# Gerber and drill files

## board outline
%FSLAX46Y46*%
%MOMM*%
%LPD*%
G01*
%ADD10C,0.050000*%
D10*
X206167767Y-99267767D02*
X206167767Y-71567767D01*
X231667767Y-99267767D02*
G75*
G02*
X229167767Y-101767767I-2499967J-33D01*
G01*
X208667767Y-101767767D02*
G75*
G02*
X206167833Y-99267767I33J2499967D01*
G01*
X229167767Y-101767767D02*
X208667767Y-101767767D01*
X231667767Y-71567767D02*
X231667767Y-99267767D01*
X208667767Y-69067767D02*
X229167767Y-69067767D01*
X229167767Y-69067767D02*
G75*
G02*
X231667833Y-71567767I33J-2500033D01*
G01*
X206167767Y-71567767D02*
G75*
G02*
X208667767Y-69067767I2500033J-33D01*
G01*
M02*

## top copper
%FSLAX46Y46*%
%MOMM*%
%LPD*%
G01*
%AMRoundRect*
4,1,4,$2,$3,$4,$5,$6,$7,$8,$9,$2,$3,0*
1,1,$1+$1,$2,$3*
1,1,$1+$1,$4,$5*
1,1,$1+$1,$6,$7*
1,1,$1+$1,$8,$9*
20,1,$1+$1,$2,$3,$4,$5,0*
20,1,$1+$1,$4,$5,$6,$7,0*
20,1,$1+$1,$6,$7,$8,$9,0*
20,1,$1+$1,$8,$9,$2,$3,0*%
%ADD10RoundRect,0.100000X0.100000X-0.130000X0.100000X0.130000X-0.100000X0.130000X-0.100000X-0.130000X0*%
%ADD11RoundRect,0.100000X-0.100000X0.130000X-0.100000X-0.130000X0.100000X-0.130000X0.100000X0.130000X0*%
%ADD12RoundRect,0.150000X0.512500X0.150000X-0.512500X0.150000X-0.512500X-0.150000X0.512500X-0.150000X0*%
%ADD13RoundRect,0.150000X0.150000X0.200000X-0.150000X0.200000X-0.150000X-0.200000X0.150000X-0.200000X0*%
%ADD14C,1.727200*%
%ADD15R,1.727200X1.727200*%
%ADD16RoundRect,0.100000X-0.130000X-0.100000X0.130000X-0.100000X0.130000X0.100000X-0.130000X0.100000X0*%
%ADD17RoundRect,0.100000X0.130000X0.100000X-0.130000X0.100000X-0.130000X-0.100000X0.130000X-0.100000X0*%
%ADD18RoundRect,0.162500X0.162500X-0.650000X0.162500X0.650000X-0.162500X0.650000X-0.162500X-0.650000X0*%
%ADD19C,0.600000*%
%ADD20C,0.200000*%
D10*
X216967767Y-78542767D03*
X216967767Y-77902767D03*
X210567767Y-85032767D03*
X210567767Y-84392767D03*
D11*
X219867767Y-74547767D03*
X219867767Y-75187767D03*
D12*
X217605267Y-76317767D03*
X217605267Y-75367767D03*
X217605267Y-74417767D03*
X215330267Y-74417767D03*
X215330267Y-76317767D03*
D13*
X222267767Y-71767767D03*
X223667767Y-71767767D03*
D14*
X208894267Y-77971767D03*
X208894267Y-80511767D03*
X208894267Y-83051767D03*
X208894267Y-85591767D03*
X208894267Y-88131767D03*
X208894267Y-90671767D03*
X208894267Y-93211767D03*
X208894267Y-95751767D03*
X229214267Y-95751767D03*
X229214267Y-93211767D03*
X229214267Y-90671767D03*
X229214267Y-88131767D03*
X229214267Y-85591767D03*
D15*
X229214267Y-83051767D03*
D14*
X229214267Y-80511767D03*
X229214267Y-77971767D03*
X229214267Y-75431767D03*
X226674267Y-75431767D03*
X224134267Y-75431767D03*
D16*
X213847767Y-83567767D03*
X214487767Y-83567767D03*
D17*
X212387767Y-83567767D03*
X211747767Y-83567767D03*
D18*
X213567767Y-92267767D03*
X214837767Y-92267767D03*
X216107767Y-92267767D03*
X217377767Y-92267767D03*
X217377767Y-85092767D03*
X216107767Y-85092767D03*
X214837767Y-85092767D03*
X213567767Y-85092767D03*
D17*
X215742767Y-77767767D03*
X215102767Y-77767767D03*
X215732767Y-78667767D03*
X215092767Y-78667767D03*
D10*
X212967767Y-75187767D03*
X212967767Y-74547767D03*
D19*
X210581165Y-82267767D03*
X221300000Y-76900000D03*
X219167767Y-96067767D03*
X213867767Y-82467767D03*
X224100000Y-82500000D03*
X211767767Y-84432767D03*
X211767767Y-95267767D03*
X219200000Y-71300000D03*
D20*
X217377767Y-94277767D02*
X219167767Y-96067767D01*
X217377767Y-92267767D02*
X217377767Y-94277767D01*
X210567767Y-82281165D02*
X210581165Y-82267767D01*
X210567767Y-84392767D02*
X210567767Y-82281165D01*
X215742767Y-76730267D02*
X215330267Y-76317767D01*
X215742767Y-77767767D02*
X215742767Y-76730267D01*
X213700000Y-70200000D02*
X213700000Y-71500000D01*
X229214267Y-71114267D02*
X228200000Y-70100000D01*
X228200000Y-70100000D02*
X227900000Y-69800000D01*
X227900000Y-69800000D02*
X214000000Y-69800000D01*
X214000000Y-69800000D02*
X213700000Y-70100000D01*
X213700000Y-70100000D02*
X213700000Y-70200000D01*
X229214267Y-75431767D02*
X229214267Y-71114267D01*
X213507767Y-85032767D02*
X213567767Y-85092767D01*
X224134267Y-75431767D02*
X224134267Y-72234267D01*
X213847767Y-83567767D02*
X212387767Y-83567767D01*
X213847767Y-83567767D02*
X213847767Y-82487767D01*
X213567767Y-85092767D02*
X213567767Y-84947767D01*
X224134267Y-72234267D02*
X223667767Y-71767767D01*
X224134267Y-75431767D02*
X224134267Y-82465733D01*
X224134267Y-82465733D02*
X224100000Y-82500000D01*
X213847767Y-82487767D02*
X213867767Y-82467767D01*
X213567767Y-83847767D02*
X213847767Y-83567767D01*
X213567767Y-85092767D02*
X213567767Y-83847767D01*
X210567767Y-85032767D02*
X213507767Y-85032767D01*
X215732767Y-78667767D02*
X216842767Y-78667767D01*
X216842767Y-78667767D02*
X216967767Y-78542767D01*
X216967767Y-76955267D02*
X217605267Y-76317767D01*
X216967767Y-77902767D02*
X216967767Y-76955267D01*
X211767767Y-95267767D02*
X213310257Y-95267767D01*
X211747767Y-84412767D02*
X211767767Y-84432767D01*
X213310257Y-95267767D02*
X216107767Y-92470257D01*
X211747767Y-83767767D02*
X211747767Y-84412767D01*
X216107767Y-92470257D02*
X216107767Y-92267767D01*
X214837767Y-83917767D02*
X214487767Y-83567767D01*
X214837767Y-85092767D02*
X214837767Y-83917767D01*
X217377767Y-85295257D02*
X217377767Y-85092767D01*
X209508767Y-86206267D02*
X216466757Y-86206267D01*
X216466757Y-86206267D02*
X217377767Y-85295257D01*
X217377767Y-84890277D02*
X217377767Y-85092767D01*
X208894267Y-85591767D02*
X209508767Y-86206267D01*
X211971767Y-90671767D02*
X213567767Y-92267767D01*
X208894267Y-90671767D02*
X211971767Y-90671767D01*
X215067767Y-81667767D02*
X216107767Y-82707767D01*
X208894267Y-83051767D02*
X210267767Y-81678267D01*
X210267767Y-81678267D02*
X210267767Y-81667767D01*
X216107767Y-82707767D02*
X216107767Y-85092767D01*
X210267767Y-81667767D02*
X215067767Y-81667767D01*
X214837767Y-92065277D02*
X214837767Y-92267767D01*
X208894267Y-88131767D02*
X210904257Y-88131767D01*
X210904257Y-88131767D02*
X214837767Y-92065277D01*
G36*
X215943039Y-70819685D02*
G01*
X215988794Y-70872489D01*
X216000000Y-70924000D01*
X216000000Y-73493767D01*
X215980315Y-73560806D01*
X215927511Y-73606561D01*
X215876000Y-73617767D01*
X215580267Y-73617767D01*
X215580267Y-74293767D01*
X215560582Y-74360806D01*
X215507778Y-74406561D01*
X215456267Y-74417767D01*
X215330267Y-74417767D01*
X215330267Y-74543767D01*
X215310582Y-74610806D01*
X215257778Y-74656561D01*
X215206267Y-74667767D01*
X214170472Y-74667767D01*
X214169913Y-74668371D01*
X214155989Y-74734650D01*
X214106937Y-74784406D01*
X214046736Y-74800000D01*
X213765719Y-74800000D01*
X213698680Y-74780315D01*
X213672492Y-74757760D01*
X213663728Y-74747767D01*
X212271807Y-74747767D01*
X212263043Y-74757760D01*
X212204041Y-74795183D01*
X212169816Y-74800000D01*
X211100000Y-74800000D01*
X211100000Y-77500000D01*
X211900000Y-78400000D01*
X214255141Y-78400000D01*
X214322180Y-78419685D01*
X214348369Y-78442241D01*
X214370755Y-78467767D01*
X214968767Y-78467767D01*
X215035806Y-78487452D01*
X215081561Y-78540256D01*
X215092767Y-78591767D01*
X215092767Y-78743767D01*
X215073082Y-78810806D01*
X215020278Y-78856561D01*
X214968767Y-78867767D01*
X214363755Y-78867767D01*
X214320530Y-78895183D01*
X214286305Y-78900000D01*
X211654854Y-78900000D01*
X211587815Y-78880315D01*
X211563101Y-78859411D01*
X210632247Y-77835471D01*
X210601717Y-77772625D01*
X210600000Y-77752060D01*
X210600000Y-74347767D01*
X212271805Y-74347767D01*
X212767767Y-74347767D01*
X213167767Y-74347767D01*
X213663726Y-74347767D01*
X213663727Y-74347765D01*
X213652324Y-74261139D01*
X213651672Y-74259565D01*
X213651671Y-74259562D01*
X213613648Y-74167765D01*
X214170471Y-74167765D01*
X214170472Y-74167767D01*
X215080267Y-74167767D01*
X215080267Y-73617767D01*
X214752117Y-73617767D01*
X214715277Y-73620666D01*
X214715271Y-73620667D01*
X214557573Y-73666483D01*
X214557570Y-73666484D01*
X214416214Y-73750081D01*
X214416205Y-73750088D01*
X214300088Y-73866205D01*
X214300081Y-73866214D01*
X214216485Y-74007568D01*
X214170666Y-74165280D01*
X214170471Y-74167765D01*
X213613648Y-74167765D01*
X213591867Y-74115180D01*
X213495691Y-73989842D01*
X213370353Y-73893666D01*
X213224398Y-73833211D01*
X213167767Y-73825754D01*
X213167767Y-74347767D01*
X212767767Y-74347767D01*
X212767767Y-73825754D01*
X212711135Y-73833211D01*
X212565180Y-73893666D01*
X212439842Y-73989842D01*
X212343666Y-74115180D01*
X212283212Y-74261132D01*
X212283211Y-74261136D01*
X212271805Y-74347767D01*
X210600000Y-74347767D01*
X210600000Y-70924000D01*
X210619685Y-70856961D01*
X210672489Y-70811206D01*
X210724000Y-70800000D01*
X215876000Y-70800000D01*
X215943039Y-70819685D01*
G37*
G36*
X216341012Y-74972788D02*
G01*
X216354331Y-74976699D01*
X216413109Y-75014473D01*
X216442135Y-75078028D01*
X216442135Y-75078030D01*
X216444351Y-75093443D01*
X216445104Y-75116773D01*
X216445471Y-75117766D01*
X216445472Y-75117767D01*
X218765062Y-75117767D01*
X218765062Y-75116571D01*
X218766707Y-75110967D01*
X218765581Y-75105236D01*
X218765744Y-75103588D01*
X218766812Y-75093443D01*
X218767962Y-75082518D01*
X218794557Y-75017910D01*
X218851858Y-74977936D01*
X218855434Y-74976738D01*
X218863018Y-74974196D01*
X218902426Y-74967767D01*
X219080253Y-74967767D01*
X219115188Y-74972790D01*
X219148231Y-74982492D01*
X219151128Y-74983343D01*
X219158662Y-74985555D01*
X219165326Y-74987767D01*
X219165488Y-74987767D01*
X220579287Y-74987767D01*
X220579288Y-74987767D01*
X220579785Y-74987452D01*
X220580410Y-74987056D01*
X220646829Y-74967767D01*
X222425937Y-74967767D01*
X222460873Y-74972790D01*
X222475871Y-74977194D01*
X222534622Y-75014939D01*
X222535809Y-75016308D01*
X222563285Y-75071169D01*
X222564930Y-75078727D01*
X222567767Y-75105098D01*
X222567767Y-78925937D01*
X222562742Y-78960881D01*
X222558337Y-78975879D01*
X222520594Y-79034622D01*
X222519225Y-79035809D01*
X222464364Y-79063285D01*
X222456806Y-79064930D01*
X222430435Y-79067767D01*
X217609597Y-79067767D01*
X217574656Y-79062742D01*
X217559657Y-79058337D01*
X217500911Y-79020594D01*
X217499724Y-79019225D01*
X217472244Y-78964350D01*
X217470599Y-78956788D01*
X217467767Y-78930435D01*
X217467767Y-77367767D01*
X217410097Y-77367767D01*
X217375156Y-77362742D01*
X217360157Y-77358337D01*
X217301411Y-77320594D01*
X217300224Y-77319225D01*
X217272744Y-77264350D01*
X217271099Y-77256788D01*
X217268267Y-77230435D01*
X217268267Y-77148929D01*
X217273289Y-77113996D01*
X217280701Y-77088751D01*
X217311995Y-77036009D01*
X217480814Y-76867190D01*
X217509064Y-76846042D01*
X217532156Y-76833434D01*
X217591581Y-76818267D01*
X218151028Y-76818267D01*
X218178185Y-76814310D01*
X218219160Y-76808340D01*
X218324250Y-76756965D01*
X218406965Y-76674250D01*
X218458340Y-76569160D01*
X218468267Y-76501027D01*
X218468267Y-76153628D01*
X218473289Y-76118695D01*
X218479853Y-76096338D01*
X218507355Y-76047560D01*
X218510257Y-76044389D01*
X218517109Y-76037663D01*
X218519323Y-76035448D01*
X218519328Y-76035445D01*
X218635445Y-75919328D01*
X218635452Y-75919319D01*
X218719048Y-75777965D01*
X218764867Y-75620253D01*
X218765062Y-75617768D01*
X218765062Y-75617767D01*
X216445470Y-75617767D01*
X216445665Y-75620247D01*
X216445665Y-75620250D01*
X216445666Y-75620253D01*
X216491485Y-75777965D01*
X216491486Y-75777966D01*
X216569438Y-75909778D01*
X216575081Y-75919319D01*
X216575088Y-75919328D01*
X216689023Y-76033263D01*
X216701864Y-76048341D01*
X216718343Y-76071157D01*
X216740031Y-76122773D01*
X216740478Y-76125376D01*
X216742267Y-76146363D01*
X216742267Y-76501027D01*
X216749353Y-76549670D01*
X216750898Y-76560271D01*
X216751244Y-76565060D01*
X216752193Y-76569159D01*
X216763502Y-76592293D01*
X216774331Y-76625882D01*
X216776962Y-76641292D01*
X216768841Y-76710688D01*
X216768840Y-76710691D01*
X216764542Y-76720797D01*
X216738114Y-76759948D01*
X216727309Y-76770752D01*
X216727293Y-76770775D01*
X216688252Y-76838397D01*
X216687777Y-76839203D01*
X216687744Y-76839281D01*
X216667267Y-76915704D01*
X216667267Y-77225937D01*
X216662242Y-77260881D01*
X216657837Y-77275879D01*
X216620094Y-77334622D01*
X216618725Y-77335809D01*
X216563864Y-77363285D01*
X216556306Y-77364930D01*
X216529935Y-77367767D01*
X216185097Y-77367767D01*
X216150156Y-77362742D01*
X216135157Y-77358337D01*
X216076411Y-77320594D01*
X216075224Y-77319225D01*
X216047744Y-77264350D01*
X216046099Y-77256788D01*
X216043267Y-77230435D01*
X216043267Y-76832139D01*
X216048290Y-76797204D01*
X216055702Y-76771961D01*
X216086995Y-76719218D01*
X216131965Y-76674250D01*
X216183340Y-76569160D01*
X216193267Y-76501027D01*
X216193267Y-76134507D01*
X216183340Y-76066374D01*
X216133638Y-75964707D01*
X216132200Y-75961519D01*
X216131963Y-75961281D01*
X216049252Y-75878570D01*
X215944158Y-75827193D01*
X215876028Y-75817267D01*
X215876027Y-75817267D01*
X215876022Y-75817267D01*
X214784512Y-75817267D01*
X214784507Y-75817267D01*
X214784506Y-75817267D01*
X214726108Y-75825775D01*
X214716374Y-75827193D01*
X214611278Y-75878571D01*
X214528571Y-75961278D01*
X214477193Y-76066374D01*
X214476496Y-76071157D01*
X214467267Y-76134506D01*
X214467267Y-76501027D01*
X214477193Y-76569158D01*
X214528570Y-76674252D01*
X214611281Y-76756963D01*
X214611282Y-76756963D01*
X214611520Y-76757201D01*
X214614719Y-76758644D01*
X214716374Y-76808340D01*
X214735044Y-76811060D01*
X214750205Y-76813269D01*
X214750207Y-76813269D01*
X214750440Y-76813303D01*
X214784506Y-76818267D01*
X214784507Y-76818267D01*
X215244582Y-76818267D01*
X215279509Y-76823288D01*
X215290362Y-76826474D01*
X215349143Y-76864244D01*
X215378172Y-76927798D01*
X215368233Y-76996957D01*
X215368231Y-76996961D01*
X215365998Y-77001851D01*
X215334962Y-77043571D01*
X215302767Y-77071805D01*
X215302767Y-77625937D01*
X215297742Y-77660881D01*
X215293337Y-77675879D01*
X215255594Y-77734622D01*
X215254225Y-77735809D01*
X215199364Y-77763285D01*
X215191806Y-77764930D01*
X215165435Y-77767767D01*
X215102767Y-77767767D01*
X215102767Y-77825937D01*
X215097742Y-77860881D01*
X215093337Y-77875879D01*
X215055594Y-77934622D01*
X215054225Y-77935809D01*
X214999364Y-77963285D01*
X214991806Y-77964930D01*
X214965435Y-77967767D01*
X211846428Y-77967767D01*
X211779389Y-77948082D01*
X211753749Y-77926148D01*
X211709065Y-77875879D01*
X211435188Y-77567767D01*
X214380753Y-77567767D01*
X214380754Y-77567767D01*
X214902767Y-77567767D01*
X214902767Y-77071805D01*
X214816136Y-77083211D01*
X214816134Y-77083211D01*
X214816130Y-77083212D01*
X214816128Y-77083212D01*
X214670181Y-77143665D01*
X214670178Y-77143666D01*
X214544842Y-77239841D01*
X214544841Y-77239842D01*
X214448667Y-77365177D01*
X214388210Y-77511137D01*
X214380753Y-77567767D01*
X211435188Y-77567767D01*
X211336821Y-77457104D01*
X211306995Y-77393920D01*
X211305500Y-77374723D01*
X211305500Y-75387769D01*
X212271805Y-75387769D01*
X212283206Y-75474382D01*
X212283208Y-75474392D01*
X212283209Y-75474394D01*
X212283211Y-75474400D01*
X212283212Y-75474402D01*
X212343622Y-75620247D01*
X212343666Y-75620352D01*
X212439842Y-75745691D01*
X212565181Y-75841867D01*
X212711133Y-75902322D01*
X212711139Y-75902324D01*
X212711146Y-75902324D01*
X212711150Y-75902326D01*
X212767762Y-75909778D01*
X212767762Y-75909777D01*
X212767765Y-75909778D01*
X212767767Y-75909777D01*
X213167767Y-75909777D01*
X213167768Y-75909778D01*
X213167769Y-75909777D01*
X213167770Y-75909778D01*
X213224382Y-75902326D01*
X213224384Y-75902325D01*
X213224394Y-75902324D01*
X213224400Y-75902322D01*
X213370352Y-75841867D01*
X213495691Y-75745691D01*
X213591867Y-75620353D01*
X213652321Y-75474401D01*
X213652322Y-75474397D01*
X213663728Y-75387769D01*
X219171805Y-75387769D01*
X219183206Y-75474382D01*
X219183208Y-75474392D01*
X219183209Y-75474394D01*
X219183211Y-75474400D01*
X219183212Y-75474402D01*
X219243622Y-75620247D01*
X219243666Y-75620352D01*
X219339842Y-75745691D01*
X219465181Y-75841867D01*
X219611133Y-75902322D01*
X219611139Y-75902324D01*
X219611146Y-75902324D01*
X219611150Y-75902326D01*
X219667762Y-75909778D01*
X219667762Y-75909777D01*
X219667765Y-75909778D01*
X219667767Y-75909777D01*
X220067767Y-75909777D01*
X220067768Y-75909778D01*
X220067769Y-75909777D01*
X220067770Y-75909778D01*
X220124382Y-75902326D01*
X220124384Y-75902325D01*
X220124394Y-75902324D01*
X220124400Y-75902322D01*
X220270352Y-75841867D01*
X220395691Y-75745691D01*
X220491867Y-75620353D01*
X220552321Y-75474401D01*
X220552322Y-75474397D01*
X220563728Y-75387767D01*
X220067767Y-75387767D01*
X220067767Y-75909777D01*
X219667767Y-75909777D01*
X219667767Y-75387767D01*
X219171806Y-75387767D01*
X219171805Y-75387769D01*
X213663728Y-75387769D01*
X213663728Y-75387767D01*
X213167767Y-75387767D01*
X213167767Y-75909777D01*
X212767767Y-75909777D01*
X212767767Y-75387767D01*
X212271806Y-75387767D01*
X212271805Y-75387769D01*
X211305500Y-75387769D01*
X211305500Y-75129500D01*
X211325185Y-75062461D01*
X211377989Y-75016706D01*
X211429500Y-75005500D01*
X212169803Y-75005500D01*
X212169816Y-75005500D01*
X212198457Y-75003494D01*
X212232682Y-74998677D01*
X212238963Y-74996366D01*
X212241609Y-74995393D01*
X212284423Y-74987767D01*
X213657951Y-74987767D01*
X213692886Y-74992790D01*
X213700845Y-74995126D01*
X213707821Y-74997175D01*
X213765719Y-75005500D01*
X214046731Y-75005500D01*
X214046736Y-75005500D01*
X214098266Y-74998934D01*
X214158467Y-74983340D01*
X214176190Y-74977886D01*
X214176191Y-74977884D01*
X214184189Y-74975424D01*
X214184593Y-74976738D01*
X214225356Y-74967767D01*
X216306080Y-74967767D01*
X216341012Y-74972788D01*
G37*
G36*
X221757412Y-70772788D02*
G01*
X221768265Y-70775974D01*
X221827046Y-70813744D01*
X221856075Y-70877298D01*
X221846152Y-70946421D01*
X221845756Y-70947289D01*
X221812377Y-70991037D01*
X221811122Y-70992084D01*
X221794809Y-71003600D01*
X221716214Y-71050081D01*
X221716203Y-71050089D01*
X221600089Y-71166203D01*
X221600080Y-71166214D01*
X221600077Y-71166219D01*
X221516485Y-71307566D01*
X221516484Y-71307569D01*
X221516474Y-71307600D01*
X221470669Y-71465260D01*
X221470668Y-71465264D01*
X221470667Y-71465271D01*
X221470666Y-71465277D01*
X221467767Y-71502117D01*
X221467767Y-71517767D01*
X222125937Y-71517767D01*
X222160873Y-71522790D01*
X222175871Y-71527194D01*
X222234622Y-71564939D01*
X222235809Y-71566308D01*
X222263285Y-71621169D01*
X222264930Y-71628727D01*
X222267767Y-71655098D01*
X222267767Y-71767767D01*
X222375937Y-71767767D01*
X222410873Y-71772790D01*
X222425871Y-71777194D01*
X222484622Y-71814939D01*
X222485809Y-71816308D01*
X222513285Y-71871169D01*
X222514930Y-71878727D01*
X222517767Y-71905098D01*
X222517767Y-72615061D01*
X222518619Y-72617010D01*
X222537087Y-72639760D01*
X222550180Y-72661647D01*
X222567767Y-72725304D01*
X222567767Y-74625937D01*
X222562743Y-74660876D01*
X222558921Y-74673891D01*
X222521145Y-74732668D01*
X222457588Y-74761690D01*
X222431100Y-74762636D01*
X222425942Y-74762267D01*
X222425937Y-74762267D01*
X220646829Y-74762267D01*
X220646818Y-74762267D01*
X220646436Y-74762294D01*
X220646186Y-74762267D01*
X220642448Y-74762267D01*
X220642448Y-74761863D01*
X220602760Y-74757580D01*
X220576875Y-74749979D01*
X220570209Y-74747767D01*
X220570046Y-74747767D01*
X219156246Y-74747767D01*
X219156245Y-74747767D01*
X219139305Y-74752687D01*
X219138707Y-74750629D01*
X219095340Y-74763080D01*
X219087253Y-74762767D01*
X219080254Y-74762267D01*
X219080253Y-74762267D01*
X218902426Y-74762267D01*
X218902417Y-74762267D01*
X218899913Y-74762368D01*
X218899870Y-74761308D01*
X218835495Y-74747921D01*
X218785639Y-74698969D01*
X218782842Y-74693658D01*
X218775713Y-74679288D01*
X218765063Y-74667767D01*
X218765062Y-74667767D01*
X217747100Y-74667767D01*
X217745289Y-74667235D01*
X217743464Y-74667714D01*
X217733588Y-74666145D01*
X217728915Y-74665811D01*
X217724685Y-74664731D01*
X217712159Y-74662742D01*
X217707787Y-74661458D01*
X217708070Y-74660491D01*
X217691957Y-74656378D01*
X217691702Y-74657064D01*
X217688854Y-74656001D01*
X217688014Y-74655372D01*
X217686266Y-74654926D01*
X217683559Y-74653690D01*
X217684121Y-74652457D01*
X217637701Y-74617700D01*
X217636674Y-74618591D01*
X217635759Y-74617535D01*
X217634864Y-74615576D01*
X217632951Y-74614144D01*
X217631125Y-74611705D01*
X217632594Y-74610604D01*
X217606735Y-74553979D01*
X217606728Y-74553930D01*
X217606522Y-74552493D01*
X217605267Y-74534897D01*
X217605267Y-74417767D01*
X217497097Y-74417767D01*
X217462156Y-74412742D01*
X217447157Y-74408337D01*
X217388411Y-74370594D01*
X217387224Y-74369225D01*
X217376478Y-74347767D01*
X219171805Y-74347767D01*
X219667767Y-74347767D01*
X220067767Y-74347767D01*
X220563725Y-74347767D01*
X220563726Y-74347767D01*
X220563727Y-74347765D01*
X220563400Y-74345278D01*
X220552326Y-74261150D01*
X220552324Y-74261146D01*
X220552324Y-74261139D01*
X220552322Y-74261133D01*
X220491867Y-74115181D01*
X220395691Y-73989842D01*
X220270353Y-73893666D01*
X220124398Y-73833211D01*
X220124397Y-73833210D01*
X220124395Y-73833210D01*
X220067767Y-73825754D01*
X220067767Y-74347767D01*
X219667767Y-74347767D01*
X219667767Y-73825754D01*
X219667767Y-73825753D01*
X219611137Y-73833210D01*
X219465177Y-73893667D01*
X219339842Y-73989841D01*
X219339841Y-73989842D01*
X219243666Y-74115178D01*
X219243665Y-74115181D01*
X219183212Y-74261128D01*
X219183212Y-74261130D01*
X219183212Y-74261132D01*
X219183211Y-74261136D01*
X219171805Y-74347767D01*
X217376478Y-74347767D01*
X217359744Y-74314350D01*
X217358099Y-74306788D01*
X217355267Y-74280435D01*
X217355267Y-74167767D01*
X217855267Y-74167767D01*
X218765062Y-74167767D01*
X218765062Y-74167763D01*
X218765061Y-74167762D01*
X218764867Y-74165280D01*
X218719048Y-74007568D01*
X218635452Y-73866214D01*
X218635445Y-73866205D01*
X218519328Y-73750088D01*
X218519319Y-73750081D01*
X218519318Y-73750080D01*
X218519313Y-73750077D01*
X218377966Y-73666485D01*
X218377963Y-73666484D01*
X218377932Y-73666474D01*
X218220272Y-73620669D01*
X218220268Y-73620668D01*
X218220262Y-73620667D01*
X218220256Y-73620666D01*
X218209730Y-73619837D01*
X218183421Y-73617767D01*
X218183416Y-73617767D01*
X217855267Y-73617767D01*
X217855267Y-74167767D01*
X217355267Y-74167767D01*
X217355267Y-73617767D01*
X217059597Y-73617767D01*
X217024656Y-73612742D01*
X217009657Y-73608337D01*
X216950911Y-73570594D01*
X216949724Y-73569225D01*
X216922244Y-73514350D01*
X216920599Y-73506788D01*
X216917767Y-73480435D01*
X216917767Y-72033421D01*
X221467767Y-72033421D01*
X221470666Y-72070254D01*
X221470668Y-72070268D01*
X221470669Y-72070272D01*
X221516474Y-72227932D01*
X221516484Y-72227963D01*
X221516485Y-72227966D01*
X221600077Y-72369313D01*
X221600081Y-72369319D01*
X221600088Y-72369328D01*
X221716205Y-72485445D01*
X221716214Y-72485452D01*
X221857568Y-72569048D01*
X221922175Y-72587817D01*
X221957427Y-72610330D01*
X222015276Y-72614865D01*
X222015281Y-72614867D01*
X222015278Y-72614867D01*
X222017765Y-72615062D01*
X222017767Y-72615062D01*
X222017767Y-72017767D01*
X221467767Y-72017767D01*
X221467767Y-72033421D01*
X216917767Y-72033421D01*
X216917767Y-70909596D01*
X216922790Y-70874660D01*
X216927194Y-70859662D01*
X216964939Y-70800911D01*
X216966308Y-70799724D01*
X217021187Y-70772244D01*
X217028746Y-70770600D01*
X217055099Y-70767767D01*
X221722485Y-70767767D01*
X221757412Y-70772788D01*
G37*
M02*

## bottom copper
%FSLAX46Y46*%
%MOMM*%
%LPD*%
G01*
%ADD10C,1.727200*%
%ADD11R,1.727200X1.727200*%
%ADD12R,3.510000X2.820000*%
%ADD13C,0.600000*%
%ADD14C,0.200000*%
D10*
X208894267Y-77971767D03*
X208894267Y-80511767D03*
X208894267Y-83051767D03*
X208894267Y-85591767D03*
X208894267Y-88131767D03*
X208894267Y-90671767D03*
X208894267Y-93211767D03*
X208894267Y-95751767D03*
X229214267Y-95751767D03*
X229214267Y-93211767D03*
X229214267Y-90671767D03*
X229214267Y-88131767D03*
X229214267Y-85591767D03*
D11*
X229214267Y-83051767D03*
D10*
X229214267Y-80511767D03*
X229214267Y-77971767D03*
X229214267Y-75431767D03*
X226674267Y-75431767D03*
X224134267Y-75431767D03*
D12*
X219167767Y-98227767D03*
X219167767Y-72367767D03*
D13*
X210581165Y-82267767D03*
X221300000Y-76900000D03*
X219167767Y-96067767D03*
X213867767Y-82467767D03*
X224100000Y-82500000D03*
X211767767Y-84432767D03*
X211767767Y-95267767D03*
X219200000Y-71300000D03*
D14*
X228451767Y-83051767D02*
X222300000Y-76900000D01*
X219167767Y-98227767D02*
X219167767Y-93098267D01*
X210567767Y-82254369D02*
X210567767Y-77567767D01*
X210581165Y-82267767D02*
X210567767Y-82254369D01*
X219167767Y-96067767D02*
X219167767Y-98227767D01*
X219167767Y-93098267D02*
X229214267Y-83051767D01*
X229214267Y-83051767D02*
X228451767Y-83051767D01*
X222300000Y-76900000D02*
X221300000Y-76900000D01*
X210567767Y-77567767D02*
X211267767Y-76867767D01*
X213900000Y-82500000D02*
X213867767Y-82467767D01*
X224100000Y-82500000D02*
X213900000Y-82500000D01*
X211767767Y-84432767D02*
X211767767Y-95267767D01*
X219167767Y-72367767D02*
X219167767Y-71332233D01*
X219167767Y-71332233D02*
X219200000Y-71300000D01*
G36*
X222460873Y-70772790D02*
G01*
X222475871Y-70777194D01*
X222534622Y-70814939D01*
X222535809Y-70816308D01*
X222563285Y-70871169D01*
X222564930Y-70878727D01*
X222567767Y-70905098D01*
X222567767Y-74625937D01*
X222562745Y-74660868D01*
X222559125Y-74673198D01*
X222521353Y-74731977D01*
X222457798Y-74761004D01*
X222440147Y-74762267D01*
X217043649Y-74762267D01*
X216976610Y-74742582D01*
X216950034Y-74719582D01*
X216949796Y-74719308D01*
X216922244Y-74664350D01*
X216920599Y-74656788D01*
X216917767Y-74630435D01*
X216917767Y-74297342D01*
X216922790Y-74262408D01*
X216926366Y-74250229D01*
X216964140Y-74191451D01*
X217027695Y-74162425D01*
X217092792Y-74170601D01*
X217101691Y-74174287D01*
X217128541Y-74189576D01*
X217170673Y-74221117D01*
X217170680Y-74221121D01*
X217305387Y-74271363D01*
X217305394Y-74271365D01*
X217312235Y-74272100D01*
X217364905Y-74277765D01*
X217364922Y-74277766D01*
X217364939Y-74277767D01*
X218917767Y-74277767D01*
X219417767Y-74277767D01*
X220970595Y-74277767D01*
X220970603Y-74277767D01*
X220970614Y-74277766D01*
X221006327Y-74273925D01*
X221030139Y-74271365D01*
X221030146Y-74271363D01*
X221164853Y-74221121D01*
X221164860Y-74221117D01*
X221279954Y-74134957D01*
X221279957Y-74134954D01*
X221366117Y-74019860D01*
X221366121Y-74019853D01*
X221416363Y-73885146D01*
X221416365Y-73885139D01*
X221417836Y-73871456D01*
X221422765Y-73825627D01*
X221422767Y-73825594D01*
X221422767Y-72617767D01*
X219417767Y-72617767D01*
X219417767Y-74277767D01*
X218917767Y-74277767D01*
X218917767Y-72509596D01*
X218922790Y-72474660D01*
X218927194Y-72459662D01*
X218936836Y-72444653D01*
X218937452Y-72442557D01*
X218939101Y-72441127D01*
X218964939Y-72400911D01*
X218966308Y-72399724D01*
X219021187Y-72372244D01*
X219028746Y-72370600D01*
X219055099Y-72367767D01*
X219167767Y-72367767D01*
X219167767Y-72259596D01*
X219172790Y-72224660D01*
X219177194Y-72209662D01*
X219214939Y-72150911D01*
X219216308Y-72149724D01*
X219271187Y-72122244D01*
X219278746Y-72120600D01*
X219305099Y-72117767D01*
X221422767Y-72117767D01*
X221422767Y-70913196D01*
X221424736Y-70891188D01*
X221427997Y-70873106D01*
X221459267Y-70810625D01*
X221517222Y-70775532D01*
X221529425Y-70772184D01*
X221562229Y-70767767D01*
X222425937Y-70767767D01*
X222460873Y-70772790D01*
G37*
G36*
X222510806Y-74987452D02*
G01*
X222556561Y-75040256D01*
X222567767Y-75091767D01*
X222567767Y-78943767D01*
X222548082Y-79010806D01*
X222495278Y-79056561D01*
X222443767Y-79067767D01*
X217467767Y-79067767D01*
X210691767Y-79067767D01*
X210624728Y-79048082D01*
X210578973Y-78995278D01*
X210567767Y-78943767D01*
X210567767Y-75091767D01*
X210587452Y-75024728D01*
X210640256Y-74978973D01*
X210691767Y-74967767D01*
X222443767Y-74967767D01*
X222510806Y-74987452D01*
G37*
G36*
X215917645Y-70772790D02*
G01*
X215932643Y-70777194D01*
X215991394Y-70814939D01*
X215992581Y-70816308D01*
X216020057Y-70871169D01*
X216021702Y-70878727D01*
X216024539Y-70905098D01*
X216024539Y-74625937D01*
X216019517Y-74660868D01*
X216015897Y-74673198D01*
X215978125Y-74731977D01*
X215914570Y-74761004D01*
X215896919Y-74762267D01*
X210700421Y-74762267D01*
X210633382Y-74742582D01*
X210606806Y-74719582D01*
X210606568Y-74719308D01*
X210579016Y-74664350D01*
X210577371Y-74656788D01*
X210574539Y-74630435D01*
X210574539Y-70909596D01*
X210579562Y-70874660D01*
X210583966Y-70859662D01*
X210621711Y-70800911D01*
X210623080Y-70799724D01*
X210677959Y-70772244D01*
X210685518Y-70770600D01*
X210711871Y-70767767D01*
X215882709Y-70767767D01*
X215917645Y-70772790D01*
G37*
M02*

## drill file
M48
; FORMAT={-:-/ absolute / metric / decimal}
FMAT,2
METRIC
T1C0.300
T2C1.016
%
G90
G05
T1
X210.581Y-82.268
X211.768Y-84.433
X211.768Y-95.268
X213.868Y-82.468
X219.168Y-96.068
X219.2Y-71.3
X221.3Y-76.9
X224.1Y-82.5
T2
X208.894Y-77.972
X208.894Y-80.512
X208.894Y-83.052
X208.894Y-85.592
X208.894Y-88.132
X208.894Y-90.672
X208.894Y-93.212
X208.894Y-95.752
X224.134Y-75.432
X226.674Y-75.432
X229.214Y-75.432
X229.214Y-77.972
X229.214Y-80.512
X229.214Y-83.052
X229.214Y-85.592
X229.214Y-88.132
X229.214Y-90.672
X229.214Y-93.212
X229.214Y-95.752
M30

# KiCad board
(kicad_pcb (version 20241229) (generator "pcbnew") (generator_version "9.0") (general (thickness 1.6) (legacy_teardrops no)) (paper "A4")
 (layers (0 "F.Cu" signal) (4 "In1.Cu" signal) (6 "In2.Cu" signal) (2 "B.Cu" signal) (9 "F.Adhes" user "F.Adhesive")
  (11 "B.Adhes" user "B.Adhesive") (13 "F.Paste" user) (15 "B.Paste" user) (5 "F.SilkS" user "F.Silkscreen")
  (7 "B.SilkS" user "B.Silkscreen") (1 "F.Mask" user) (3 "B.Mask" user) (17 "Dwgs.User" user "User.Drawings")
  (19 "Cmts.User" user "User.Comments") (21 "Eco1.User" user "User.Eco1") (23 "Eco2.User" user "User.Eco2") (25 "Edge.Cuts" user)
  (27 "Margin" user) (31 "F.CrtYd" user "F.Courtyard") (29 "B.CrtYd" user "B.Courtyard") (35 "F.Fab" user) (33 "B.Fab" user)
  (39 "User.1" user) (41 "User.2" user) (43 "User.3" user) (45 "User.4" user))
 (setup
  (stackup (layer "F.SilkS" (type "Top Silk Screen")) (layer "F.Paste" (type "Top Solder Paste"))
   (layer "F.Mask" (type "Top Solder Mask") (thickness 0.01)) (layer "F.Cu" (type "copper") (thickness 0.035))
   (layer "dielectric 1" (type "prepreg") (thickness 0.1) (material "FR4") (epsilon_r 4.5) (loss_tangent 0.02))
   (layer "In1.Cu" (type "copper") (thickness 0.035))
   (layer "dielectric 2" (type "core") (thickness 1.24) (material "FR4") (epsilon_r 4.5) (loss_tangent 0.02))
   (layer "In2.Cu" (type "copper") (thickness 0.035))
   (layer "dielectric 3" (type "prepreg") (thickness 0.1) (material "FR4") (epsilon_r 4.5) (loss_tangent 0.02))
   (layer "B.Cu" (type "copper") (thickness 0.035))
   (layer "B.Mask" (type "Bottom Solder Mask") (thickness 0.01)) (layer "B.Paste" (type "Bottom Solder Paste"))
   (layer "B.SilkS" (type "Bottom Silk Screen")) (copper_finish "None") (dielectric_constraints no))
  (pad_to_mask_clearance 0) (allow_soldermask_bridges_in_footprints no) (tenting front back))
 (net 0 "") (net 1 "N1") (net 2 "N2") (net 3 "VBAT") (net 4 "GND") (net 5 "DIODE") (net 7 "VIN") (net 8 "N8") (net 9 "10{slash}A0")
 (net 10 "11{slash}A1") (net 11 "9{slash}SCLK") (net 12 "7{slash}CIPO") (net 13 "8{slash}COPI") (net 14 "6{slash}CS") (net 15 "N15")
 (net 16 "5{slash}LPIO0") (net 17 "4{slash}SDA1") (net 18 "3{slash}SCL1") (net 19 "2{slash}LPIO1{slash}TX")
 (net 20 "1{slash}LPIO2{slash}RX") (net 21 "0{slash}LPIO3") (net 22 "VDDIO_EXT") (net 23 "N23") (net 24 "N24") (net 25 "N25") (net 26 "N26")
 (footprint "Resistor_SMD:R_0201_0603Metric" (layer "F.Cu") (at 216.967767 78.222767 90)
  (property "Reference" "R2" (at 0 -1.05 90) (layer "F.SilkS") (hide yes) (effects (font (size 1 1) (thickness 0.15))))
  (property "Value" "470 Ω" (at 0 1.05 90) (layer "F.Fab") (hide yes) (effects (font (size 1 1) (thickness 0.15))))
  (pad "" smd roundrect (at -0.345 0 90) (size 0.318 0.36) (layers "F.Paste") (roundrect_rratio 0.25))
  (pad "" smd roundrect (at 0.345 0 90) (size 0.318 0.36) (layers "F.Paste") (roundrect_rratio 0.25))
  (pad "1" smd roundrect (at -0.32 0 90) (size 0.46 0.4) (layers "F.Cu" "F.Mask") (roundrect_rratio 0.25) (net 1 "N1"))
  (pad "2" smd roundrect (at 0.32 0 90) (size 0.46 0.4) (layers "F.Cu" "F.Mask") (roundrect_rratio 0.25) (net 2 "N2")))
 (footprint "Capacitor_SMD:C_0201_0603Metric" (layer "F.Cu") (at 210.567767 84.712767 90)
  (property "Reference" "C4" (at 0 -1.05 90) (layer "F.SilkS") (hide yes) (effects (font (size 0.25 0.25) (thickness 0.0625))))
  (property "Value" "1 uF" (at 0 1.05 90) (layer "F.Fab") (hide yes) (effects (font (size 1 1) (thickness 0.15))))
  (pad "" smd roundrect (at -0.345 0 90) (size 0.318 0.36) (layers "F.Paste") (roundrect_rratio 0.25))
  (pad "" smd roundrect (at 0.345 0 90) (size 0.318 0.36) (layers "F.Paste") (roundrect_rratio 0.25))
  (pad "1" smd roundrect (at -0.32 0 90) (size 0.46 0.4) (layers "F.Cu" "F.Mask") (roundrect_rratio 0.25) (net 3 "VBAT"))
  (pad "2" smd roundrect (at 0.32 0 90) (size 0.46 0.4) (layers "F.Cu" "F.Mask") (roundrect_rratio 0.25) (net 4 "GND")))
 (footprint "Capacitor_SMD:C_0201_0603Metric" (layer "F.Cu") (at 219.867767 74.867767 -90)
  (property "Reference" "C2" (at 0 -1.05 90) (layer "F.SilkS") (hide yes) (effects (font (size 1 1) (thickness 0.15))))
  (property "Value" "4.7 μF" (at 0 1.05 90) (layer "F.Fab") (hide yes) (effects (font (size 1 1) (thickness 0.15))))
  (pad "" smd roundrect (at -0.345 0 270) (size 0.318 0.36) (layers "F.Paste") (roundrect_rratio 0.25))
  (pad "" smd roundrect (at 0.345 0 270) (size 0.318 0.36) (layers "F.Paste") (roundrect_rratio 0.25))
  (pad "1" smd roundrect (at -0.32 0 270) (size 0.46 0.4) (layers "F.Cu" "F.Mask") (roundrect_rratio 0.25) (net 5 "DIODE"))
  (pad "2" smd roundrect (at 0.32 0 270) (size 0.46 0.4) (layers "F.Cu" "F.Mask") (roundrect_rratio 0.25) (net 4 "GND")))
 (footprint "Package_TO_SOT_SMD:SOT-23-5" (layer "F.Cu") (at 216.467767 75.367767 180)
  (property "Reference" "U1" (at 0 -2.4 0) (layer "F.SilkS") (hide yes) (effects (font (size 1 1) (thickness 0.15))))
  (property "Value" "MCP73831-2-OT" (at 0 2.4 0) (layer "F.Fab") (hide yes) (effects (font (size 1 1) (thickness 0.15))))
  (pad "1" smd roundrect (at -1.1375 -0.95 180) (size 1.325 0.6) (layers "F.Cu" "F.Mask" "F.Paste") (roundrect_rratio 0.25) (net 2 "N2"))
  (pad "2" smd roundrect (at -1.1375 0 180) (size 1.325 0.6) (layers "F.Cu" "F.Mask" "F.Paste") (roundrect_rratio 0.25) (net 4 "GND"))
  (pad "3" smd roundrect (at -1.1375 0.95 180) (size 1.325 0.6) (layers "F.Cu" "F.Mask" "F.Paste") (roundrect_rratio 0.25) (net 5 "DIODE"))
  (pad "4" smd roundrect (at 1.1375 0.95 180) (size 1.325 0.6) (layers "F.Cu" "F.Mask" "F.Paste") (roundrect_rratio 0.25) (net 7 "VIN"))
  (pad "5" smd roundrect (at 1.1375 -0.95 180) (size 1.325 0.6) (layers "F.Cu" "F.Mask" "F.Paste") (roundrect_rratio 0.25) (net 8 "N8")))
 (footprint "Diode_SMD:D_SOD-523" (layer "F.Cu") (at 222.967767 71.767767)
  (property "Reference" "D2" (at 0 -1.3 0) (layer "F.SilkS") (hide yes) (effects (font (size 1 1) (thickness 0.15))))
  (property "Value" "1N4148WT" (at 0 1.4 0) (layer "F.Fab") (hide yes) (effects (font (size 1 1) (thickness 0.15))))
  (pad "1" smd roundrect (at -0.7 0 180) (size 0.6 0.7) (layers "F.Cu" "F.Mask" "F.Paste") (roundrect_rratio 0.25) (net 5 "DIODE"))
  (pad "2" smd roundrect (at 0.7 0 180) (size 0.6 0.7) (layers "F.Cu" "F.Mask" "F.Paste") (roundrect_rratio 0.25) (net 3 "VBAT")))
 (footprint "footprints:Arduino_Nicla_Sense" (layer "F.Cu") (at 207.624267 74.161767)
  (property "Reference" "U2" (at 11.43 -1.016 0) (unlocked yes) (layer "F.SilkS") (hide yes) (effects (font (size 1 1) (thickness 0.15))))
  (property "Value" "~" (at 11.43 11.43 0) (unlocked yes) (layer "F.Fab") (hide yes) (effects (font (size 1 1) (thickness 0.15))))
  (pad "1" thru_hole circle (at 1.27 3.81) (size 1.7272 1.7272) (drill 1.016) (layers "*.Cu" "*.Mask") (remove_unused_layers no)
   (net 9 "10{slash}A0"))
  (pad "2" thru_hole circle (at 1.27 6.35) (size 1.7272 1.7272) (drill 1.016) (layers "*.Cu" "*.Mask") (remove_unused_layers no)
   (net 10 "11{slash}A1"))
  (pad "3" thru_hole circle (at 1.27 8.89) (size 1.7272 1.7272) (drill 1.016) (layers "*.Cu" "*.Mask") (remove_unused_layers no)
   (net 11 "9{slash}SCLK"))
  (pad "4" thru_hole circle (at 1.27 11.43) (size 1.7272 1.7272) (drill 1.016) (layers "*.Cu" "*.Mask") (remove_unused_layers no)
   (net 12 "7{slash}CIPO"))
  (pad "5" thru_hole circle (at 1.27 13.97) (size 1.7272 1.7272) (drill 1.016) (layers "*.Cu" "*.Mask") (remove_unused_layers no)
   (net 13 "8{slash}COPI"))
  (pad "6" thru_hole circle (at 1.27 16.51) (size 1.7272 1.7272) (drill 1.016) (layers "*.Cu" "*.Mask") (remove_unused_layers no)
   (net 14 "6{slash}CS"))
  (pad "7" thru_hole circle (at 1.27 19.05) (size 1.7272 1.7272) (drill 1.016) (layers "*.Cu" "*.Mask") (remove_unused_layers no)
   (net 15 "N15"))
  (pad "8" thru_hole circle (at 1.27 21.59) (size 1.7272 1.7272) (drill 1.016) (layers "*.Cu" "*.Mask") (remove_unused_layers no)
   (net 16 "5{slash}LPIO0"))
  (pad "9" thru_hole circle (at 21.59 21.59) (size 1.7272 1.7272) (drill 1.016) (layers "*.Cu" "*.Mask") (remove_unused_layers no)
   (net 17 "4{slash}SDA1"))
  (pad "10" thru_hole circle (at 21.59 19.05) (size 1.7272 1.7272) (drill 1.016) (layers "*.Cu" "*.Mask") (remove_unused_layers no)
   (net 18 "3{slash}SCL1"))
  (pad "11" thru_hole circle (at 21.59 16.51) (size 1.7272 1.7272) (drill 1.016) (layers "*.Cu" "*.Mask") (remove_unused_layers no)
   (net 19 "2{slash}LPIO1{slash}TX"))
  (pad "12" thru_hole circle (at 21.59 13.97) (size 1.7272 1.7272) (drill 1.016) (layers "*.Cu" "*.Mask") (remove_unused_layers no)
   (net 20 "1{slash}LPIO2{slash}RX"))
  (pad "13" thru_hole circle (at 21.59 11.43) (size 1.7272 1.7272) (drill 1.016) (layers "*.Cu" "*.Mask") (remove_unused_layers no)
   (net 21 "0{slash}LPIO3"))
  (pad "14" thru_hole rect (at 21.59 8.89) (size 1.7272 1.7272) (drill 1.016) (layers "*.Cu" "*.Mask") (remove_unused_layers no)
   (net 4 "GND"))
  (pad "15" thru_hole circle (at 21.59 6.35) (size 1.7272 1.7272) (drill 1.016) (layers "*.Cu" "*.Mask") (remove_unused_layers no)
   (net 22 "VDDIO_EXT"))
  (pad "16" thru_hole circle (at 21.59 3.81) (size 1.7272 1.7272) (drill 1.016) (layers "*.Cu" "*.Mask") (remove_unused_layers no)
   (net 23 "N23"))
  (pad "17" thru_hole circle (at 21.59 1.27) (size 1.7272 1.7272) (drill 1.016) (layers "*.Cu" "*.Mask") (remove_unused_layers no)
   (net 7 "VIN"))
  (pad "18" thru_hole circle (at 19.05 1.27) (size 1.7272 1.7272) (drill 1.016) (layers "*.Cu" "*.Mask") (remove_unused_layers no)
   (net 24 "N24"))
  (pad "19" thru_hole circle (at 16.51 1.27) (size 1.7272 1.7272) (drill 1.016) (layers "*.Cu" "*.Mask") (remove_unused_layers no)
   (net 3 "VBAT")))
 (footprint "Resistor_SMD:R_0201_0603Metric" (layer "F.Cu") (at 214.167767 83.567767)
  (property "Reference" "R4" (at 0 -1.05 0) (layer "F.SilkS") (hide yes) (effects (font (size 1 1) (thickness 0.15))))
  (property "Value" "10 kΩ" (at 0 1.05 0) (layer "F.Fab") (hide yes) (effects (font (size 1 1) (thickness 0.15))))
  (pad "" smd roundrect (at -0.345 0) (size 0.318 0.36) (layers "F.Paste") (roundrect_rratio 0.25))
  (pad "" smd roundrect (at 0.345 0) (size 0.318 0.36) (layers "F.Paste") (roundrect_rratio 0.25))
  (pad "1" smd roundrect (at -0.32 0) (size 0.46 0.4) (layers "F.Cu" "F.Mask") (roundrect_rratio 0.25) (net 3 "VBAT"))
  (pad "2" smd roundrect (at 0.32 0) (size 0.46 0.4) (layers "F.Cu" "F.Mask") (roundrect_rratio 0.25) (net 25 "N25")))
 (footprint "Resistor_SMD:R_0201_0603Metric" (layer "F.Cu") (at 212.067767 83.567767 180)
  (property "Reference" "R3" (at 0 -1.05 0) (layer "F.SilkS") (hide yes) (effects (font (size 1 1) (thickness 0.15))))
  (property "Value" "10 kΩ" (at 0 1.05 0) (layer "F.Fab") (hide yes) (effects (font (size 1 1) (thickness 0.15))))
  (pad "" smd roundrect (at -0.345 0 180) (size 0.318 0.36) (layers "F.Paste") (roundrect_rratio 0.25))
  (pad "" smd roundrect (at 0.345 0 180) (size 0.318 0.36) (layers "F.Paste") (roundrect_rratio 0.25))
  (pad "1" smd roundrect (at -0.32 0 180) (size 0.46 0.4) (layers "F.Cu" "F.Mask") (roundrect_rratio 0.25) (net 3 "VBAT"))
  (pad "2" smd roundrect (at 0.32 0 180) (size 0.46 0.4) (layers "F.Cu" "F.Mask") (roundrect_rratio 0.25) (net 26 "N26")))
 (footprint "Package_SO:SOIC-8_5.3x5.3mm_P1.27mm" (layer "F.Cu") (at 215.472767 88.680267 90)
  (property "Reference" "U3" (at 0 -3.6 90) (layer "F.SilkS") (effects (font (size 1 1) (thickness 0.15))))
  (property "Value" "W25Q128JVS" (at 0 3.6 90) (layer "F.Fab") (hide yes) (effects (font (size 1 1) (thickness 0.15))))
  (pad "1" smd roundrect (at -3.5875 -1.905 90) (size 1.625 0.65) (layers "F.Cu" "F.Mask" "F.Paste") (roundrect_rratio 0.25)
   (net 14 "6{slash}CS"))
  (pad "2" smd roundrect (at -3.5875 -0.635 90) (size 1.625 0.65) (layers "F.Cu" "F.Mask" "F.Paste") (roundrect_rratio 0.25)
   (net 13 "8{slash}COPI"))
  (pad "3" smd roundrect (at -3.5875 0.635 90) (size 1.625 0.65) (layers "F.Cu" "F.Mask" "F.Paste") (roundrect_rratio 0.25) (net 26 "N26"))
  (pad "4" smd roundrect (at -3.5875 1.905 90) (size 1.625 0.65) (layers "F.Cu" "F.Mask" "F.Paste") (roundrect_rratio 0.25) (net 4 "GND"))
  (pad "5" smd roundrect (at 3.5875 1.905 90) (size 1.625 0.65) (layers "F.Cu" "F.Mask" "F.Paste") (roundrect_rratio 0.25)
   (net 12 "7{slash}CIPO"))
  (pad "6" smd roundrect (at 3.5875 0.635 90) (size 1.625 0.65) (layers "F.Cu" "F.Mask" "F.Paste") (roundrect_rratio 0.25)
   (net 11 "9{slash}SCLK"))
  (pad "7" smd roundrect (at 3.5875 -0.635 90) (size 1.625 0.65) (layers "F.Cu" "F.Mask" "F.Paste") (roundrect_rratio 0.25) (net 25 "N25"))
  (pad "8" smd roundrect (at 3.5875 -1.905 90) (size 1.625 0.65) (layers "F.Cu" "F.Mask" "F.Paste") (roundrect_rratio 0.25) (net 3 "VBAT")))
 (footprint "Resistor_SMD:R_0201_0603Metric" (layer "F.Cu") (at 215.422767 77.767767 180)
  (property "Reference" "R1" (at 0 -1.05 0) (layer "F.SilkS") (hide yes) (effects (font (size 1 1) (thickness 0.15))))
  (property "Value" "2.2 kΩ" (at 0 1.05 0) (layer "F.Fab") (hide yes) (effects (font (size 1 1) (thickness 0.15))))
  (pad "" smd roundrect (at -0.345 0 180) (size 0.318 0.36) (layers "F.Paste") (roundrect_rratio 0.25))
  (pad "" smd roundrect (at 0.345 0 180) (size 0.318 0.36) (layers "F.Paste") (roundrect_rratio 0.25))
  (pad "1" smd roundrect (at -0.32 0 180) (size 0.46 0.4) (layers "F.Cu" "F.Mask") (roundrect_rratio 0.25) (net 8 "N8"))
  (pad "2" smd roundrect (at 0.32 0 180) (size 0.46 0.4) (layers "F.Cu" "F.Mask") (roundrect_rratio 0.25) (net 4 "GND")))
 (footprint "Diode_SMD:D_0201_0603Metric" (layer "F.Cu") (at 215.412767 78.667767 180)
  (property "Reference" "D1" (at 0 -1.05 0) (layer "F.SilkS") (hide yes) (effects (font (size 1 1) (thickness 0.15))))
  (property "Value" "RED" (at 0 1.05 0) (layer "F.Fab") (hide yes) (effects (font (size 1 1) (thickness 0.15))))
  (pad "" smd roundrect (at -0.345 0 180) (size 0.318 0.36) (layers "F.Paste") (roundrect_rratio 0.25))
  (pad "" smd roundrect (at 0.345 0 180) (size 0.318 0.36) (layers "F.Paste") (roundrect_rratio 0.25))
  (pad "1" smd roundrect (at -0.32 0 180) (size 0.46 0.4) (layers "F.Cu" "F.Mask") (roundrect_rratio 0.25) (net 1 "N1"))
  (pad "2" smd roundrect (at 0.32 0 180) (size 0.46 0.4) (layers "F.Cu" "F.Mask") (roundrect_rratio 0.25) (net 7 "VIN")))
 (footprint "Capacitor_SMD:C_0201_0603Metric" (layer "F.Cu") (at 212.967767 74.867767 90)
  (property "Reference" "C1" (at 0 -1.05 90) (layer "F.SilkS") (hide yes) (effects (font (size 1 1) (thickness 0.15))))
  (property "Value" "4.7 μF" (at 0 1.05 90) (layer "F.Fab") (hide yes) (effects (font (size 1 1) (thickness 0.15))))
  (pad "" smd roundrect (at -0.345 0 90) (size 0.318 0.36) (layers "F.Paste") (roundrect_rratio 0.25))
  (pad "" smd roundrect (at 0.345 0 90) (size 0.318 0.36) (layers "F.Paste") (roundrect_rratio 0.25))
  (pad "1" smd roundrect (at -0.32 0 90) (size 0.46 0.4) (layers "F.Cu" "F.Mask") (roundrect_rratio 0.25) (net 4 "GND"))
  (pad "2" smd roundrect (at 0.32 0 90) (size 0.46 0.4) (layers "F.Cu" "F.Mask") (roundrect_rratio 0.25) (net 7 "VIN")))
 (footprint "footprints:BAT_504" (layer "B.Cu") (at 219.167767 85.297767 -90)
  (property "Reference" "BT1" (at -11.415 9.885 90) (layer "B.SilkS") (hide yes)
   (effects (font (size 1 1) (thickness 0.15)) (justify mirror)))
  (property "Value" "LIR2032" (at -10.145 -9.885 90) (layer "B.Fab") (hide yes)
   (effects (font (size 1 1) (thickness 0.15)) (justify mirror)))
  (pad "N" smd rect (at 12.93 0 270) (size 2.82 3.51) (layers "B.Cu" "B.Mask" "B.Paste") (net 4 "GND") (solder_mask_margin 0.102))
  (pad "P" smd rect (at -12.93 0 270) (size 2.82 3.51) (layers "B.Cu" "B.Mask" "B.Paste") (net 5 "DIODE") (solder_mask_margin 0.102)))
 (gr_line (start 206.167767 99.267767) (end 206.167767 71.567767) (stroke (width 0.05) (type default)) (layer "Edge.Cuts"))
 (gr_arc (start 231.667767 99.267767) (mid 230.935534 101.035534) (end 229.167767 101.767767) (stroke (width 0.05) (type default))
  (layer "Edge.Cuts"))
 (gr_arc (start 208.667767 101.767767) (mid 206.9 101.035534) (end 206.167767 99.267767) (stroke (width 0.05) (type default))
  (layer "Edge.Cuts"))
 (gr_line (start 229.167767 101.767767) (end 208.667767 101.767767) (stroke (width 0.05) (type default)) (layer "Edge.Cuts"))
 (gr_line (start 231.667767 71.567767) (end 231.667767 99.267767) (stroke (width 0.05) (type default)) (layer "Edge.Cuts"))
 (gr_line (start 208.667767 69.067767) (end 229.167767 69.067767) (stroke (width 0.05) (type default)) (layer "Edge.Cuts"))
 (gr_arc (start 229.167767 69.067767) (mid 230.935534 69.8) (end 231.667767 71.567767) (stroke (width 0.05) (type default))
  (layer "Edge.Cuts"))
 (gr_arc (start 206.167767 71.567767) (mid 206.9 69.8) (end 208.667767 69.067767) (stroke (width 0.05) (type default)) (layer "Edge.Cuts"))
 (segment (start 217.377767 94.277767) (end 219.167767 96.067767) (width 0.2) (layer "F.Cu") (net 4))
 (segment (start 217.377767 92.267767) (end 217.377767 94.277767) (width 0.2) (layer "F.Cu") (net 4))
 (segment (start 210.567767 82.281165) (end 210.581165 82.267767) (width 0.2) (layer "F.Cu") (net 4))
 (segment (start 210.567767 84.392767) (end 210.567767 82.281165) (width 0.2) (layer "F.Cu") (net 4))
 (via (at 210.581165 82.267767) (size 0.6) (drill 0.3) (layers "F.Cu" "B.Cu") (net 4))
 (via (at 221.3 76.9) (size 0.6) (drill 0.3) (layers "F.Cu" "B.Cu") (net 4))
 (via (at 219.167767 96.067767) (size 0.6) (drill 0.3) (layers "F.Cu" "B.Cu") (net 4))
 (segment (start 228.451767 83.051767) (end 222.3 76.9) (width 0.2) (layer "B.Cu") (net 4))
 (segment (start 219.167767 98.227767) (end 219.167767 93.098267) (width 0.2) (layer "B.Cu") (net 4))
 (segment (start 210.567767 82.254369) (end 210.567767 77.567767) (width 0.2) (layer "B.Cu") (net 4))
 (segment (start 210.581165 82.267767) (end 210.567767 82.254369) (width 0.2) (layer "B.Cu") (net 4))
 (segment (start 219.167767 96.067767) (end 219.167767 98.227767) (width 0.2) (layer "B.Cu") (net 4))
 (segment (start 219.167767 93.098267) (end 229.214267 83.051767) (width 0.2) (layer "B.Cu") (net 4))
 (segment (start 229.214267 83.051767) (end 228.451767 83.051767) (width 0.2) (layer "B.Cu") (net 4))
 (segment (start 222.3 76.9) (end 221.3 76.9) (width 0.2) (layer "B.Cu") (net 4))
 (segment (start 210.567767 77.567767) (end 211.267767 76.867767) (width 0.2) (layer "B.Cu") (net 4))
 (segment (start 215.742767 76.730267) (end 215.330267 76.317767) (width 0.2) (layer "F.Cu") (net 8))
 (segment (start 215.742767 77.767767) (end 215.742767 76.730267) (width 0.2) (layer "F.Cu") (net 8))
 (segment (start 213.7 70.2) (end 213.7 71.5) (width 0.2) (layer "F.Cu") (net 7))
 (segment (start 229.214267 71.114267) (end 228.2 70.1) (width 0.2) (layer "F.Cu") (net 7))
 (segment (start 228.2 70.1) (end 227.9 69.8) (width 0.2) (layer "F.Cu") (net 7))
 (segment (start 227.9 69.8) (end 214 69.8) (width 0.2) (layer "F.Cu") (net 7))
 (segment (start 214 69.8) (end 213.7 70.1) (width 0.2) (layer "F.Cu") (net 7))
 (segment (start 213.7 70.1) (end 213.7 70.2) (width 0.2) (layer "F.Cu") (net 7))
 (segment (start 229.214267 75.431767) (end 229.214267 71.114267) (width 0.2) (layer "F.Cu") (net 7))
 (segment (start 213.507767 85.032767) (end 213.567767 85.092767) (width 0.2) (layer "F.Cu") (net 3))
 (segment (start 224.134267 75.431767) (end 224.134267 72.234267) (width 0.2) (layer "F.Cu") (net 3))
 (segment (start 213.847767 83.567767) (end 212.387767 83.567767) (width 0.2) (layer "F.Cu") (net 3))
 (segment (start 213.847767 83.567767) (end 213.847767 82.487767) (width 0.2) (layer "F.Cu") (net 3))
 (segment (start 213.567767 85.092767) (end 213.567767 84.947767) (width 0.2) (layer "F.Cu") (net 3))
 (segment (start 224.134267 72.234267) (end 223.667767 71.767767) (width 0.2) (layer "F.Cu") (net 3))
 (segment (start 224.134267 75.431767) (end 224.134267 82.465733) (width 0.2) (layer "F.Cu") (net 3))
 (segment (start 224.134267 82.465733) (end 224.1 82.5) (width 0.2) (layer "F.Cu") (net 3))
 (segment (start 213.847767 82.487767) (end 213.867767 82.467767) (width 0.2) (layer "F.Cu") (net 3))
 (segment (start 213.567767 83.847767) (end 213.847767 83.567767) (width 0.2) (layer "F.Cu") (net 3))
 (segment (start 213.567767 85.092767) (end 213.567767 83.847767) (width 0.2) (layer "F.Cu") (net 3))
 (segment (start 210.567767 85.032767) (end 213.507767 85.032767) (width 0.2) (layer "F.Cu") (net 3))
 (via (at 213.867767 82.467767) (size 0.6) (drill 0.3) (layers "F.Cu" "B.Cu") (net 3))
 (via (at 224.1 82.5) (size 0.6) (drill 0.3) (layers "F.Cu" "B.Cu") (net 3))
 (segment (start 213.9 82.5) (end 213.867767 82.467767) (width 0.2) (layer "B.Cu") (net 3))
 (segment (start 224.1 82.5) (end 213.9 82.5) (width 0.2) (layer "B.Cu") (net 3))
 (segment (start 215.732767 78.667767) (end 216.842767 78.667767) (width 0.2) (layer "F.Cu") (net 1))
 (segment (start 216.842767 78.667767) (end 216.967767 78.542767) (width 0.2) (layer "F.Cu") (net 1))
 (segment (start 216.967767 76.955267) (end 217.605267 76.317767) (width 0.2) (layer "F.Cu") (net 2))
 (segment (start 216.967767 77.902767) (end 216.967767 76.955267) (width 0.2) (layer "F.Cu") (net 2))
 (segment (start 211.767767 95.267767) (end 213.310257 95.267767) (width 0.2) (layer "F.Cu") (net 26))
 (segment (start 211.747767 84.412767) (end 211.767767 84.432767) (width 0.2) (layer "F.Cu") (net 26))
 (segment (start 213.310257 95.267767) (end 216.107767 92.470257) (width 0.2) (layer "F.Cu") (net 26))
 (segment (start 211.747767 83.767767) (end 211.747767 84.412767) (width 0.2) (layer "F.Cu") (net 26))
 (segment (start 216.107767 92.470257) (end 216.107767 92.267767) (width 0.2) (layer "F.Cu") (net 26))
 (via (at 211.767767 84.432767) (size 0.6) (drill 0.3) (layers "F.Cu" "B.Cu") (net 26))
 (via (at 211.767767 95.267767) (size 0.6) (drill 0.3) (layers "F.Cu" "B.Cu") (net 26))
 (segment (start 211.767767 84.432767) (end 211.767767 95.267767) (width 0.2) (layer "B.Cu") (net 26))
 (segment (start 214.837767 83.917767) (end 214.487767 83.567767) (width 0.2) (layer "F.Cu") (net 25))
 (segment (start 214.837767 85.092767) (end 214.837767 83.917767) (width 0.2) (layer "F.Cu") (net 25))
 (segment (start 217.377767 85.295257) (end 217.377767 85.092767) (width 0.2) (layer "F.Cu") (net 12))
 (segment (start 209.508767 86.206267) (end 216.466757 86.206267) (width 0.2) (layer "F.Cu") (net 12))
 (segment (start 216.466757 86.206267) (end 217.377767 85.295257) (width 0.2) (layer "F.Cu") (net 12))
 (segment (start 217.377767 84.890277) (end 217.377767 85.092767) (width 0.2) (layer "F.Cu") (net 12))
 (segment (start 208.894267 85.591767) (end 209.508767 86.206267) (width 0.2) (layer "F.Cu") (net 12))
 (segment (start 211.971767 90.671767) (end 213.567767 92.267767) (width 0.2) (layer "F.Cu") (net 14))
 (segment (start 208.894267 90.671767) (end 211.971767 90.671767) (width 0.2) (layer "F.Cu") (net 14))
 (segment (start 215.067767 81.667767) (end 216.107767 82.707767) (width 0.2) (layer "F.Cu") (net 11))
 (segment (start 208.894267 83.051767) (end 210.267767 81.678267) (width 0.2) (layer "F.Cu") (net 11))
 (segment (start 210.267767 81.678267) (end 210.267767 81.667767) (width 0.2) (layer "F.Cu") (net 11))
 (segment (start 216.107767 82.707767) (end 216.107767 85.092767) (width 0.2) (layer "F.Cu") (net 11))
 (segment (start 210.267767 81.667767) (end 215.067767 81.667767) (width 0.2) (layer "F.Cu") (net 11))
 (segment (start 214.837767 92.065277) (end 214.837767 92.267767) (width 0.2) (layer "F.Cu") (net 13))
 (segment (start 208.894267 88.131767) (end 210.904257 88.131767) (width 0.2) (layer "F.Cu") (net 13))
 (segment (start 210.904257 88.131767) (end 214.837767 92.065277) (width 0.2) (layer "F.Cu") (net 13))
 (via (at 219.2 71.3) (size 0.6) (drill 0.3) (layers "F.Cu" "B.Cu") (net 5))
 (segment (start 219.167767 72.367767) (end 219.167767 71.332233) (width 0.2) (layer "B.Cu") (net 5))
 (segment (start 219.167767 71.332233) (end 219.2 71.3) (width 0.2) (layer "B.Cu") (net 5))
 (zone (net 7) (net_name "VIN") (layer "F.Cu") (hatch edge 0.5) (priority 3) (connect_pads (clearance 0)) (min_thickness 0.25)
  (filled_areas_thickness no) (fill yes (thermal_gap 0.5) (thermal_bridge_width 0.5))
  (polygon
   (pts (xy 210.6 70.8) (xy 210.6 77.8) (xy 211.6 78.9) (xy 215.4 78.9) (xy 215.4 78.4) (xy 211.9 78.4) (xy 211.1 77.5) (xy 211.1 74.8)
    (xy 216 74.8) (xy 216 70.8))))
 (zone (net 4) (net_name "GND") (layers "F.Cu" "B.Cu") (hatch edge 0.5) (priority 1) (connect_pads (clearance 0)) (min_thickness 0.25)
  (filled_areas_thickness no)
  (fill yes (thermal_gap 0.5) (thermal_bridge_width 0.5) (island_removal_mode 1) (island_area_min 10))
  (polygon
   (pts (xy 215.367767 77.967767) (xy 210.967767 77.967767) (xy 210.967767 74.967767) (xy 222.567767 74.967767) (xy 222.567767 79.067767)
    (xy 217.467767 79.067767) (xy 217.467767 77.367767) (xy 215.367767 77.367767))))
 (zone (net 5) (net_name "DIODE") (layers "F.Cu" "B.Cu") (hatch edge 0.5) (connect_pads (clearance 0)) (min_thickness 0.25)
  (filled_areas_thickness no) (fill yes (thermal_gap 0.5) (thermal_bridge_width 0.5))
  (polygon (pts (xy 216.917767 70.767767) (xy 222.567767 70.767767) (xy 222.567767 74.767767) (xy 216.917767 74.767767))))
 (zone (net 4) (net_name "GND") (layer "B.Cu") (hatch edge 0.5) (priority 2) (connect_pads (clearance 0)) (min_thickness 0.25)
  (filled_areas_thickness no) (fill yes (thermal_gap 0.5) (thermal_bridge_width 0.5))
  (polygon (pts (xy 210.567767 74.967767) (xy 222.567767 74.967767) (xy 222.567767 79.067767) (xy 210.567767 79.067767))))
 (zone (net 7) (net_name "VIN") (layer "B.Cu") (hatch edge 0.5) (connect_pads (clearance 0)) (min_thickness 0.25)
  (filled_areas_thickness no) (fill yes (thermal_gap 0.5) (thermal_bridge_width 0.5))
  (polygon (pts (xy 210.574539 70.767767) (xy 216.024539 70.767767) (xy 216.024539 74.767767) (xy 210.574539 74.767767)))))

